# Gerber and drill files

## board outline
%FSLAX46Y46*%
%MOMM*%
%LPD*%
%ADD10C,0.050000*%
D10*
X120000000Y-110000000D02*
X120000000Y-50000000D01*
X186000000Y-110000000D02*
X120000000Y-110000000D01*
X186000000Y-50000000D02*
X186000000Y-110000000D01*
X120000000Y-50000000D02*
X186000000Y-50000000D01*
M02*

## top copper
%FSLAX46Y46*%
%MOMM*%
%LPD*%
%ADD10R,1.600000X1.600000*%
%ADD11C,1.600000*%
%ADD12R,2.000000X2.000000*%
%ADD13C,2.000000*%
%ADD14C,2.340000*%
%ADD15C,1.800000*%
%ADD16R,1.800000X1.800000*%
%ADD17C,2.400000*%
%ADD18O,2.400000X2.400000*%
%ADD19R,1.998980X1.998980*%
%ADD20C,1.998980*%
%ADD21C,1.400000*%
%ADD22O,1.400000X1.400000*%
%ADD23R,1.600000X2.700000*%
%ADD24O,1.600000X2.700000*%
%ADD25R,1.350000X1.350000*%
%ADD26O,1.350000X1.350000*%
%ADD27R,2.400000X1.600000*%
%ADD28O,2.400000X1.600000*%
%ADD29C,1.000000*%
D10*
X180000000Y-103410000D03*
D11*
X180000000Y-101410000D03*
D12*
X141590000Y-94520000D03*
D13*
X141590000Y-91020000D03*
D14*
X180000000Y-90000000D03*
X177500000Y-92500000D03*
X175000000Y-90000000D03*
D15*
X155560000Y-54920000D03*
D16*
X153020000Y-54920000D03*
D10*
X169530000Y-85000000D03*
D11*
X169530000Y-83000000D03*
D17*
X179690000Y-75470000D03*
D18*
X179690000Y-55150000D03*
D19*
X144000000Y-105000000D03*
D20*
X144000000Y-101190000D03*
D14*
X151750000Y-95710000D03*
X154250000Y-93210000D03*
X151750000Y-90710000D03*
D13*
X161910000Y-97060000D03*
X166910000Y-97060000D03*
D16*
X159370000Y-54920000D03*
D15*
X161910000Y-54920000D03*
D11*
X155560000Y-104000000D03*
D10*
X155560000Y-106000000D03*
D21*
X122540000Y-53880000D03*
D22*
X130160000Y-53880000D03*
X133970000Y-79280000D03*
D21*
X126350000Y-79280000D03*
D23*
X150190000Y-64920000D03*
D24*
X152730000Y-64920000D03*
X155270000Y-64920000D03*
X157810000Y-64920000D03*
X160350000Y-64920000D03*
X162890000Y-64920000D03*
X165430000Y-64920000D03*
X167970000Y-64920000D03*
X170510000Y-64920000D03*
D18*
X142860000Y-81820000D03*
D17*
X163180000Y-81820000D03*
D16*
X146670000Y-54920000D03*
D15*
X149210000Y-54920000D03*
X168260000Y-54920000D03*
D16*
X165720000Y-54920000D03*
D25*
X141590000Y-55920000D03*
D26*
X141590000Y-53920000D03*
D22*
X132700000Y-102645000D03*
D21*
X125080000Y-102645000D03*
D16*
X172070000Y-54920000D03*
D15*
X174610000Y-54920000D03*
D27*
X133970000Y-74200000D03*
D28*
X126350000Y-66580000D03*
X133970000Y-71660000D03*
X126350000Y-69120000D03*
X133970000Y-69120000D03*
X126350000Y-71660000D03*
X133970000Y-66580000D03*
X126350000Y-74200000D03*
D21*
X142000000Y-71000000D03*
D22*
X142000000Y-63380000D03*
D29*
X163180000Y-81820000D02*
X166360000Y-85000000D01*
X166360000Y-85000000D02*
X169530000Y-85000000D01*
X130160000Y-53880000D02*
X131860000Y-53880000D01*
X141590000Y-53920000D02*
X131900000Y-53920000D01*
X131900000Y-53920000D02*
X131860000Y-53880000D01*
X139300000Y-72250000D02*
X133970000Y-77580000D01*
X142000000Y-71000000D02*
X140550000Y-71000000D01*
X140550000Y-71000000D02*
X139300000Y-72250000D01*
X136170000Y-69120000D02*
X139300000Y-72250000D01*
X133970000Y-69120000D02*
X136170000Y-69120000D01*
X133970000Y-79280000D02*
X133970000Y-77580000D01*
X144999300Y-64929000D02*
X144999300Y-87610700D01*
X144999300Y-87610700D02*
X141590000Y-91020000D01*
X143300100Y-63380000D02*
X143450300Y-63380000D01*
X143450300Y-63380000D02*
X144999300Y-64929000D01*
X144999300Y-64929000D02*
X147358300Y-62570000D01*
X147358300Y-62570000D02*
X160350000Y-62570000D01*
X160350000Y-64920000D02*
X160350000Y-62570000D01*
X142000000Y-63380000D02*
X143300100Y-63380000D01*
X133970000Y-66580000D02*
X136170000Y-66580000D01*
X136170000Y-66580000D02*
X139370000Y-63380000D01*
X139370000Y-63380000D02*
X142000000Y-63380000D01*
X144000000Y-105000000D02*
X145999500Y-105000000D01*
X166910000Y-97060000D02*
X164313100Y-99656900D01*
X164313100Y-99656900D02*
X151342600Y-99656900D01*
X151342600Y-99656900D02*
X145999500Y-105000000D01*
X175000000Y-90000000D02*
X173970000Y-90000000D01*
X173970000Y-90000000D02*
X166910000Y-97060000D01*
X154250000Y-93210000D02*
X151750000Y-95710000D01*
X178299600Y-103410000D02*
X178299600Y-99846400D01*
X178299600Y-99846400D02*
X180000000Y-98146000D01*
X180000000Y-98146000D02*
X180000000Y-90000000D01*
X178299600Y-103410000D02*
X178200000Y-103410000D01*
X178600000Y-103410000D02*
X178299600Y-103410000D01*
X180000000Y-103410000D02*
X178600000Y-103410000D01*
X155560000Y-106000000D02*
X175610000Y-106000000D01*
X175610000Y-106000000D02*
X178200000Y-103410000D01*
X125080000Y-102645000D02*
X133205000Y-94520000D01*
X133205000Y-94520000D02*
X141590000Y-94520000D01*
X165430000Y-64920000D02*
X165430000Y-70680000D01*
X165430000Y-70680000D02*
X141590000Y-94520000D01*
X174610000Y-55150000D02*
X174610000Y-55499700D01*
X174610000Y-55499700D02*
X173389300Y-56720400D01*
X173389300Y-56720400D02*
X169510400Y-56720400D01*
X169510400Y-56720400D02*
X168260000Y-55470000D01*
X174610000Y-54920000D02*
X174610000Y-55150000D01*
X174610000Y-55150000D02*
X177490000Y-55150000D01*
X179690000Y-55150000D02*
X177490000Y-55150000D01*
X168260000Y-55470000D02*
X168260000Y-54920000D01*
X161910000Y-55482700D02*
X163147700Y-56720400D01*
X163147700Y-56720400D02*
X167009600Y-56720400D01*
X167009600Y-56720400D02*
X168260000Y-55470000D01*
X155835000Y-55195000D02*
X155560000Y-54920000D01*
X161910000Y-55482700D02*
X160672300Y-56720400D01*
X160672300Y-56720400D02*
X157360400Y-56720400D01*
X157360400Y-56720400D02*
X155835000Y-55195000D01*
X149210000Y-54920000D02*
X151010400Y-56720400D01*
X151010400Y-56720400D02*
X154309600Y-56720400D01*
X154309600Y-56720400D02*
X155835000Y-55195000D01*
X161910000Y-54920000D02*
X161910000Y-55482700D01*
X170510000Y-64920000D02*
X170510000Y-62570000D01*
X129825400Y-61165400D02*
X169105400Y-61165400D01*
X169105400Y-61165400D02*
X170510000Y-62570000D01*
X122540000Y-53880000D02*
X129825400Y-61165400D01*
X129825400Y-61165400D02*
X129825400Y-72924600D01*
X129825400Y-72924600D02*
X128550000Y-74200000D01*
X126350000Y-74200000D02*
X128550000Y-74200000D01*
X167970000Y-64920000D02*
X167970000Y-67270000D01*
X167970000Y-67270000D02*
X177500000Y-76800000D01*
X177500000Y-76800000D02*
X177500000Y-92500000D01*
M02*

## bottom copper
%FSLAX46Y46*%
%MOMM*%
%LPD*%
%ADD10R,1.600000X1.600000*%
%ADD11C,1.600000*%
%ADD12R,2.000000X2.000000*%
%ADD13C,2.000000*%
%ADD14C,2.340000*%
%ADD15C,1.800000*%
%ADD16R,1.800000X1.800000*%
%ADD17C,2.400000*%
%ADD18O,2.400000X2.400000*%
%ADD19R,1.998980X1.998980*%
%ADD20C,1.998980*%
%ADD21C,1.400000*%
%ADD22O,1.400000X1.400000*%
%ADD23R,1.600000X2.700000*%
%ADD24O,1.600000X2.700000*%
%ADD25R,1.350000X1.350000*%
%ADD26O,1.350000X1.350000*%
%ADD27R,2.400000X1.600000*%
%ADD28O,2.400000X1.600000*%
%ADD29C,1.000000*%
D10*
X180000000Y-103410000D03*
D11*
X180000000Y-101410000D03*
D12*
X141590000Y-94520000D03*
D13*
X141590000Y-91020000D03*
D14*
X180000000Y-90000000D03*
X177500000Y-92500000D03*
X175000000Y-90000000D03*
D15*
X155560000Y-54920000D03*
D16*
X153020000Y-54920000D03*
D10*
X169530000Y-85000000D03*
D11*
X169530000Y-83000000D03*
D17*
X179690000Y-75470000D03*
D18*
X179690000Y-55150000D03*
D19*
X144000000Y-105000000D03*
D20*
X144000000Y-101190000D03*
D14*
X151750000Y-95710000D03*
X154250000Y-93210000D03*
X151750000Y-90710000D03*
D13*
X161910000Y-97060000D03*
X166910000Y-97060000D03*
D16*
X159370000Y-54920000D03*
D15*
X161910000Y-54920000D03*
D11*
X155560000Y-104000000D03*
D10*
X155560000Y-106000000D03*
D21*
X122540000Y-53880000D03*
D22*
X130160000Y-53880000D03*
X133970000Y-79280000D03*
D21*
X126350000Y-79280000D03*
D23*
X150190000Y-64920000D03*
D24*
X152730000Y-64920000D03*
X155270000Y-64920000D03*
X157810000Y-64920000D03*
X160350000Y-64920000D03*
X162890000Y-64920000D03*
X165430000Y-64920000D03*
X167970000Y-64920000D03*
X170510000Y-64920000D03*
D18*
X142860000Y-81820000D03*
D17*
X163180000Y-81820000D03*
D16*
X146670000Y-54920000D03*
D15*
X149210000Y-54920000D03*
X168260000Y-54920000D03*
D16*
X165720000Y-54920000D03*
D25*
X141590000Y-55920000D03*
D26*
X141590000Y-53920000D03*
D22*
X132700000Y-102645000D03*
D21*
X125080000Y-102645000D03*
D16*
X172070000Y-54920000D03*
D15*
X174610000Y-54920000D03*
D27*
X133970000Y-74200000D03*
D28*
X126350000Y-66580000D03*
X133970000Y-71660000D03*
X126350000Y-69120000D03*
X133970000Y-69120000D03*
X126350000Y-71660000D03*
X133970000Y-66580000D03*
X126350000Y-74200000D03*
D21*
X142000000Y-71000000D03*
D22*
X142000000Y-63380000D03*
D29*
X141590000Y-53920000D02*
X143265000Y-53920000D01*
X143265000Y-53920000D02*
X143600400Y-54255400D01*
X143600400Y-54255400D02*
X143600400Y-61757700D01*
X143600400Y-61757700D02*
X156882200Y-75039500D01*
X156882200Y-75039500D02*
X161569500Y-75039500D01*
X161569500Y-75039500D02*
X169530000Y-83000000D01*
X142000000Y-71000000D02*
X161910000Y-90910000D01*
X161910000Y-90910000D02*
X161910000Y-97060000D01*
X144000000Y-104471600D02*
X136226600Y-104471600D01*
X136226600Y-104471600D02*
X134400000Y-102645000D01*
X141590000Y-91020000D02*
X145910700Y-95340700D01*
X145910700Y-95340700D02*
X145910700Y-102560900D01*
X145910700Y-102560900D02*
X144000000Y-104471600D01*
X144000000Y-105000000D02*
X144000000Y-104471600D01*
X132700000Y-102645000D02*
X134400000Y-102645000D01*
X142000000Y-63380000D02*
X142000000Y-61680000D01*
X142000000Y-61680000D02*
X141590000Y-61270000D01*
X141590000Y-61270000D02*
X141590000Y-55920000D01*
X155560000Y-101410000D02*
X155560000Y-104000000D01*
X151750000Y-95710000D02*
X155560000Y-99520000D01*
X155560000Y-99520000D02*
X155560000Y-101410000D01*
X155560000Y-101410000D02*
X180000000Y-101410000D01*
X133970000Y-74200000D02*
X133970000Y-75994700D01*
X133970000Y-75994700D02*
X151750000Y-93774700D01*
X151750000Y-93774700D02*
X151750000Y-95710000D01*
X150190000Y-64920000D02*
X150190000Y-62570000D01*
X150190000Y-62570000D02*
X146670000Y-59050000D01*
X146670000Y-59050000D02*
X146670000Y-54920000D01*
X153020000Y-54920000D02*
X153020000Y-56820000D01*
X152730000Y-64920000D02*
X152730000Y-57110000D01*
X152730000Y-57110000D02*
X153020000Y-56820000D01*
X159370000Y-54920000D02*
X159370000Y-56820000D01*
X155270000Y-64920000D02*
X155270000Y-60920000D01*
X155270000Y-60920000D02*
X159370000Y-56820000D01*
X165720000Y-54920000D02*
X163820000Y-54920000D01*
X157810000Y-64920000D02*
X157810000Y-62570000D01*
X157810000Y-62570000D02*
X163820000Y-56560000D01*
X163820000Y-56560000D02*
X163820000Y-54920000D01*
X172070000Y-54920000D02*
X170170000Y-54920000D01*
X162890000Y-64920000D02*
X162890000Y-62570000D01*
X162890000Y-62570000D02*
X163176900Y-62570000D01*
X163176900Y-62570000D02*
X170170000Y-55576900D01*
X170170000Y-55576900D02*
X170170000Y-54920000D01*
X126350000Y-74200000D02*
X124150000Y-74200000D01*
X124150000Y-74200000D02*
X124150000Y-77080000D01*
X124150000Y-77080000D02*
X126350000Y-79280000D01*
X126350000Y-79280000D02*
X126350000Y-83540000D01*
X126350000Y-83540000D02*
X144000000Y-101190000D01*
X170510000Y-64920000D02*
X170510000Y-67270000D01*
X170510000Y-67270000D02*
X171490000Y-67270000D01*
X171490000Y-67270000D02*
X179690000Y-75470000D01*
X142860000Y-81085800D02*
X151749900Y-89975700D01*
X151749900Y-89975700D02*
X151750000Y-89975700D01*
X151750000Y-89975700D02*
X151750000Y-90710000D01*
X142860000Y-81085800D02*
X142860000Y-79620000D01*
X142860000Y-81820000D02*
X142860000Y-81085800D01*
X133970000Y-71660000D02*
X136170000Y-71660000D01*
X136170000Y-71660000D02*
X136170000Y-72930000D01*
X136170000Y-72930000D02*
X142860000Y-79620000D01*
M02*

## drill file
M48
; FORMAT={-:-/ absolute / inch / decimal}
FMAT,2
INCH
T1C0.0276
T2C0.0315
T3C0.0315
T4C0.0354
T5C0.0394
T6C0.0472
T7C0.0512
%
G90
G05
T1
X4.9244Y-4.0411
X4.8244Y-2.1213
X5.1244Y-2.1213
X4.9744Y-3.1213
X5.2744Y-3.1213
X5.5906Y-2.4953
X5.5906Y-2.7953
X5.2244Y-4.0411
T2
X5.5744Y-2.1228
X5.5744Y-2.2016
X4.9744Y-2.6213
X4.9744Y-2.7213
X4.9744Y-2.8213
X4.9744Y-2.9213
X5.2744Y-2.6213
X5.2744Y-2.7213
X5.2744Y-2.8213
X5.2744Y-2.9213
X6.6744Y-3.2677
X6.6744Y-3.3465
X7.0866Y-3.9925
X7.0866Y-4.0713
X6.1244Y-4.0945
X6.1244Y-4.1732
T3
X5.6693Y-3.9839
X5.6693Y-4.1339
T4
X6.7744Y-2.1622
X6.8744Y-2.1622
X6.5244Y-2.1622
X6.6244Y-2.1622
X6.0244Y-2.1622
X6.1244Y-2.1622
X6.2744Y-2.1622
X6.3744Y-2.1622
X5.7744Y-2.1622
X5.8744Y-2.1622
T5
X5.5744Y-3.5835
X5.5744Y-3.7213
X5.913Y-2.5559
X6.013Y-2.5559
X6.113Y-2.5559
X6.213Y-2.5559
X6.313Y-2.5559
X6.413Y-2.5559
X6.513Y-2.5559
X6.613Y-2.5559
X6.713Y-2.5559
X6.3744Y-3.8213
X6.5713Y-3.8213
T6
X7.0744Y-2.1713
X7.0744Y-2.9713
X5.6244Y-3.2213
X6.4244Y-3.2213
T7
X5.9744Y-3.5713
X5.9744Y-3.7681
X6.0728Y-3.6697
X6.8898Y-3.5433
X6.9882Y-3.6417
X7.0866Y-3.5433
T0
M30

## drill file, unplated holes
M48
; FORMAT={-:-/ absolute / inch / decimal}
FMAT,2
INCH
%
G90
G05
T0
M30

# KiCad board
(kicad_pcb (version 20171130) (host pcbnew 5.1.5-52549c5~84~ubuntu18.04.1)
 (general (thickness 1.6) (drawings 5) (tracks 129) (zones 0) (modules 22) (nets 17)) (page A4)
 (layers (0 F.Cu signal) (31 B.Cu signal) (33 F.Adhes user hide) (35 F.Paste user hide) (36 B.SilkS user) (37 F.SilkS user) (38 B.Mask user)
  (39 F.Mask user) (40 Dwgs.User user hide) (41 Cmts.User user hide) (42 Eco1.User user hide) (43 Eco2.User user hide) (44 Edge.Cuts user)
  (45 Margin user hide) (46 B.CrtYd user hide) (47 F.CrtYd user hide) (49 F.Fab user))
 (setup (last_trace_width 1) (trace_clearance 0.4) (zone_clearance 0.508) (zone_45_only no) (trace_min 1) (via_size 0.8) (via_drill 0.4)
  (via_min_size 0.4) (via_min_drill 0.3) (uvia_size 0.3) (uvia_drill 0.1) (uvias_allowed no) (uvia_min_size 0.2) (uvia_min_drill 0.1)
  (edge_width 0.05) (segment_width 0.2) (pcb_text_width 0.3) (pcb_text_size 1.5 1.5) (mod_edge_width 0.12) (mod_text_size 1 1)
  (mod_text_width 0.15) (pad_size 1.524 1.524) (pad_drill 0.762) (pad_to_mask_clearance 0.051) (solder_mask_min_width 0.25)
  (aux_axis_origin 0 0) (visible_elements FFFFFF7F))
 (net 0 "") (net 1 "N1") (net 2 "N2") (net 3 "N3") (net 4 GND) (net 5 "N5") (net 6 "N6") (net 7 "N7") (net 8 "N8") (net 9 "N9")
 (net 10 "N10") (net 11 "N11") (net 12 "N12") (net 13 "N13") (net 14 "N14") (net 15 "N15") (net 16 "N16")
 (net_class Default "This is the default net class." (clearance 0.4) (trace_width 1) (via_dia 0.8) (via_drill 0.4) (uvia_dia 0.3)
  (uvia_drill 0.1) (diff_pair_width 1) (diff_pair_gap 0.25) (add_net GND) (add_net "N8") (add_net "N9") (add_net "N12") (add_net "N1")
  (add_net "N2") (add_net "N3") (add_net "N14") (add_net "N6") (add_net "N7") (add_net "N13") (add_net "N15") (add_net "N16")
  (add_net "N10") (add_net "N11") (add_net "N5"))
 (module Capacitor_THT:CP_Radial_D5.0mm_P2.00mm (layer F.Cu) (at 180 103.41 90)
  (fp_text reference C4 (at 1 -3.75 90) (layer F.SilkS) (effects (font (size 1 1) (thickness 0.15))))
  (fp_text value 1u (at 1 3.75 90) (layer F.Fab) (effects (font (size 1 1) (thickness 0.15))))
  (pad 1 thru_hole rect (at 0 0 90) (size 1.6 1.6) (drill 0.8) (layers *.Cu *.Mask) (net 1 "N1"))
  (pad 2 thru_hole circle (at 2 0 90) (size 1.6 1.6) (drill 0.8) (layers *.Cu *.Mask) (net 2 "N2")))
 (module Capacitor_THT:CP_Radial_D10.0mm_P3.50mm (layer F.Cu) (at 141.59 94.52 90)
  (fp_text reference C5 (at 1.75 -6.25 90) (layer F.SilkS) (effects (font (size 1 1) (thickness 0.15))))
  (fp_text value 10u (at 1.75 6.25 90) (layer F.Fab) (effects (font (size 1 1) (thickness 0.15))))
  (pad 1 thru_hole rect (at 0 0 90) (size 2 2) (drill 1) (layers *.Cu *.Mask) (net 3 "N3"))
  (pad 2 thru_hole circle (at 3.5 0 90) (size 2 2) (drill 1) (layers *.Cu *.Mask) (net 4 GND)))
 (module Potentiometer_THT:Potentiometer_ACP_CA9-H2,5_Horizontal (layer F.Cu) (at 180 90 270)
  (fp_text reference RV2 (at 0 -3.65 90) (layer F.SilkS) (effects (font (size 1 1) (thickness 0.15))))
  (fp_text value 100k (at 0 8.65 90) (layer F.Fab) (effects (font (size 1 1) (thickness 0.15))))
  (pad 1 thru_hole circle (at 0 0 270) (size 2.34 2.34) (drill 1.3) (layers *.Cu *.Mask) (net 1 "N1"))
  (pad 2 thru_hole circle (at 2.5 2.5 270) (size 2.34 2.34) (drill 1.3) (layers *.Cu *.Mask) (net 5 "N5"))
  (pad 3 thru_hole circle (at 0 5 270) (size 2.34 2.34) (drill 1.3) (layers *.Cu *.Mask) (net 4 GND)))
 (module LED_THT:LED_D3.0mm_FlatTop (layer F.Cu) (at 153.02 54.92)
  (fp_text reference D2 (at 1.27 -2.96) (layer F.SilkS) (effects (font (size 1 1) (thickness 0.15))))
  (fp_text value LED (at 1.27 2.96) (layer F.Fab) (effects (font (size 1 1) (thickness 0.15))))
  (pad 2 thru_hole circle (at 2.54 0) (size 1.8 1.8) (drill 0.9) (layers *.Cu *.Mask) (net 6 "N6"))
  (pad 1 thru_hole rect (at 0 0) (size 1.8 1.8) (drill 0.9) (layers *.Cu *.Mask) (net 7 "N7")))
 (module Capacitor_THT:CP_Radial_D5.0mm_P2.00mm (layer F.Cu) (at 169.53 85 90)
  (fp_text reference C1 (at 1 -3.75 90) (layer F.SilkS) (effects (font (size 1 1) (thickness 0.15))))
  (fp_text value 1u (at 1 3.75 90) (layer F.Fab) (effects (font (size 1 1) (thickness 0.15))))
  (pad 1 thru_hole rect (at 0 0 90) (size 1.6 1.6) (drill 0.8) (layers *.Cu *.Mask) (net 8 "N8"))
  (pad 2 thru_hole circle (at 2 0 90) (size 1.6 1.6) (drill 0.8) (layers *.Cu *.Mask) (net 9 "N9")))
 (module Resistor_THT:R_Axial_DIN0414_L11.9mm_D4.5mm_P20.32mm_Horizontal (layer F.Cu) (at 179.69 75.47 90)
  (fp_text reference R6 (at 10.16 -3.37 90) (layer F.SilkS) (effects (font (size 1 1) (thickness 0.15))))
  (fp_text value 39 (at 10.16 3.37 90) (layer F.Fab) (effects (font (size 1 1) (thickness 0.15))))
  (pad 1 thru_hole circle (at 0 0 90) (size 2.4 2.4) (drill 1.2) (layers *.Cu *.Mask) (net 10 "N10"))
  (pad 2 thru_hole oval (at 20.32 0 90) (size 2.4 2.4) (drill 1.2) (layers *.Cu *.Mask) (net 6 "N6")))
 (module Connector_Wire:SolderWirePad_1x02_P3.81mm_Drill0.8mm (layer F.Cu) (at 144 105 90)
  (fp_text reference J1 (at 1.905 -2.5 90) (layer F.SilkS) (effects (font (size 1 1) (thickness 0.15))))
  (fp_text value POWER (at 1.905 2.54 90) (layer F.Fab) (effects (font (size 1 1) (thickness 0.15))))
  (pad 1 thru_hole rect (at 0 0 90) (size 1.99898 1.99898) (drill 0.8001) (layers *.Cu *.Mask) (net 4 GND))
  (pad 2 thru_hole circle (at 3.81 0 90) (size 1.99898 1.99898) (drill 0.8001) (layers *.Cu *.Mask) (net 10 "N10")))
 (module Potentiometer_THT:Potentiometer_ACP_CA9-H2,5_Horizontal (layer F.Cu) (at 151.75 90.71)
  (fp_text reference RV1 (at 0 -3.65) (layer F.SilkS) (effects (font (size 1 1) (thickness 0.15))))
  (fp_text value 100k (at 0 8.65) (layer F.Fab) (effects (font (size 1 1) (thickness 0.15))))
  (pad 3 thru_hole circle (at 0 5) (size 2.34 2.34) (drill 1.3) (layers *.Cu *.Mask) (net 2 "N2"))
  (pad 2 thru_hole circle (at 2.5 2.5) (size 2.34 2.34) (drill 1.3) (layers *.Cu *.Mask) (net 2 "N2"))
  (pad 1 thru_hole circle (at 0 0) (size 2.34 2.34) (drill 1.3) (layers *.Cu *.Mask) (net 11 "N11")))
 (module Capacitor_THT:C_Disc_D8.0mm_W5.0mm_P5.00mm (layer F.Cu) (at 161.91 97.06)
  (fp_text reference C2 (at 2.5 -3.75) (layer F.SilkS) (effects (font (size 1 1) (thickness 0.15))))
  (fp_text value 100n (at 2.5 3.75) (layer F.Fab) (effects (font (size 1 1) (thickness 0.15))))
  (pad 1 thru_hole circle (at 0 0) (size 2 2) (drill 1) (layers *.Cu *.Mask) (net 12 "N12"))
  (pad 2 thru_hole circle (at 5 0) (size 2 2) (drill 1) (layers *.Cu *.Mask) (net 4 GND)))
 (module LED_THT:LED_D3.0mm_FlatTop (layer F.Cu) (at 159.37 54.92)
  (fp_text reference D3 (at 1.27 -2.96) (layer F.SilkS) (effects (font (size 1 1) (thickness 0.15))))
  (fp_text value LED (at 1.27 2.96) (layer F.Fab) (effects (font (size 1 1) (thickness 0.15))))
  (pad 1 thru_hole rect (at 0 0) (size 1.8 1.8) (drill 0.9) (layers *.Cu *.Mask) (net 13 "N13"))
  (pad 2 thru_hole circle (at 2.54 0) (size 1.8 1.8) (drill 0.9) (layers *.Cu *.Mask) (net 6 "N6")))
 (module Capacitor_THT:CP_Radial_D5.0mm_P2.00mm (layer F.Cu) (at 155.56 106 90)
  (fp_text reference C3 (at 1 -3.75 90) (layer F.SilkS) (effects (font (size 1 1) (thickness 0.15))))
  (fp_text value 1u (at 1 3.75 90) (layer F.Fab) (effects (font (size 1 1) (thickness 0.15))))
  (pad 2 thru_hole circle (at 2 0 90) (size 1.6 1.6) (drill 0.8) (layers *.Cu *.Mask) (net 2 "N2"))
  (pad 1 thru_hole rect (at 0 0 90) (size 1.6 1.6) (drill 0.8) (layers *.Cu *.Mask) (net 1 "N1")))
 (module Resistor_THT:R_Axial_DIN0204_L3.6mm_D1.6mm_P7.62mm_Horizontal (layer F.Cu) (at 122.54 53.88)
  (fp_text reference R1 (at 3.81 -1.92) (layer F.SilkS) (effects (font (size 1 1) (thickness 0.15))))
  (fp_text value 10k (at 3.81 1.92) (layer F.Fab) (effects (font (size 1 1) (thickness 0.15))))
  (pad 1 thru_hole circle (at 0 0) (size 1.4 1.4) (drill 0.7) (layers *.Cu *.Mask) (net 10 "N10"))
  (pad 2 thru_hole oval (at 7.62 0) (size 1.4 1.4) (drill 0.7) (layers *.Cu *.Mask) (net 9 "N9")))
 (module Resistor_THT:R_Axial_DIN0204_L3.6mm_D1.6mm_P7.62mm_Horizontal (layer F.Cu) (at 126.35 79.28)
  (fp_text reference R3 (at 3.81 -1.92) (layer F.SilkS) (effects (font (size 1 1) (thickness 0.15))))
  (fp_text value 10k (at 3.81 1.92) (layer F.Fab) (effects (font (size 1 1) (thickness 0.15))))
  (pad 2 thru_hole oval (at 7.62 0) (size 1.4 1.4) (drill 0.7) (layers *.Cu *.Mask) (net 12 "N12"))
  (pad 1 thru_hole circle (at 0 0) (size 1.4 1.4) (drill 0.7) (layers *.Cu *.Mask) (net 10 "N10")))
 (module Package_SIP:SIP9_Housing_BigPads (layer F.Cu) (at 150.19 64.92)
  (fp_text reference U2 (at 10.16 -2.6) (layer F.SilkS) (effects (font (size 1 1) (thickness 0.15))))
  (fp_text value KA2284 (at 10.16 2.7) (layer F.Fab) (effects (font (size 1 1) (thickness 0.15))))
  (pad 1 thru_hole rect (at 0 0 90) (size 2.7 1.6) (drill 1) (layers *.Cu *.Mask) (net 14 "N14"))
  (pad 2 thru_hole oval (at 2.54 0 90) (size 2.7 1.6) (drill 1) (layers *.Cu *.Mask) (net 7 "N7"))
  (pad 3 thru_hole oval (at 5.08 0 90) (size 2.7 1.6) (drill 1) (layers *.Cu *.Mask) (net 13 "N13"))
  (pad 4 thru_hole oval (at 7.62 0 90) (size 2.7 1.6) (drill 1) (layers *.Cu *.Mask) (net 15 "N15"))
  (pad 5 thru_hole oval (at 10.16 0 90) (size 2.7 1.6) (drill 1) (layers *.Cu *.Mask) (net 4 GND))
  (pad 6 thru_hole oval (at 12.7 0 90) (size 2.7 1.6) (drill 1) (layers *.Cu *.Mask) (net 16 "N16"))
  (pad 7 thru_hole oval (at 15.24 0 90) (size 2.7 1.6) (drill 1) (layers *.Cu *.Mask) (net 3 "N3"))
  (pad 8 thru_hole oval (at 17.78 0 90) (size 2.7 1.6) (drill 1) (layers *.Cu *.Mask) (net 5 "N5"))
  (pad 9 thru_hole oval (at 20.32 0 90) (size 2.7 1.6) (drill 1) (layers *.Cu *.Mask) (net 10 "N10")))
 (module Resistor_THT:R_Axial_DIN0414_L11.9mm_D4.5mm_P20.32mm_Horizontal (layer F.Cu) (at 163.18 81.82 180)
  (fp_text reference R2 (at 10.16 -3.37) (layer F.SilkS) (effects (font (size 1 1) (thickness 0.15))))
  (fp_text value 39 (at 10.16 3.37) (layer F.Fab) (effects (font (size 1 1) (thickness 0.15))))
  (pad 2 thru_hole oval (at 20.32 0 180) (size 2.4 2.4) (drill 1.2) (layers *.Cu *.Mask) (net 11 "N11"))
  (pad 1 thru_hole circle (at 0 0 180) (size 2.4 2.4) (drill 1.2) (layers *.Cu *.Mask) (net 8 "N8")))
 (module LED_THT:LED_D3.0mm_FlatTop (layer F.Cu) (at 146.67 54.92)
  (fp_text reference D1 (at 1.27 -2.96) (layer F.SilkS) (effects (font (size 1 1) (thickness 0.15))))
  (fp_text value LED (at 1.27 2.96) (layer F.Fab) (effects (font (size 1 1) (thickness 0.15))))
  (pad 1 thru_hole rect (at 0 0) (size 1.8 1.8) (drill 0.9) (layers *.Cu *.Mask) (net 14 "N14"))
  (pad 2 thru_hole circle (at 2.54 0) (size 1.8 1.8) (drill 0.9) (layers *.Cu *.Mask) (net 6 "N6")))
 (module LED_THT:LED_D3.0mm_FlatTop (layer F.Cu) (at 165.72 54.92)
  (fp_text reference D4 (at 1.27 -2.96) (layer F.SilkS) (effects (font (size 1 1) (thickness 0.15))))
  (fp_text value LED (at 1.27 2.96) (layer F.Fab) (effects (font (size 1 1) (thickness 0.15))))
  (pad 2 thru_hole circle (at 2.54 0) (size 1.8 1.8) (drill 0.9) (layers *.Cu *.Mask) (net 6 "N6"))
  (pad 1 thru_hole rect (at 0 0) (size 1.8 1.8) (drill 0.9) (layers *.Cu *.Mask) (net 15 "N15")))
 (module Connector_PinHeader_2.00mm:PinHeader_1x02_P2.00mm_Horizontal (layer F.Cu) (at 141.59 55.92 180)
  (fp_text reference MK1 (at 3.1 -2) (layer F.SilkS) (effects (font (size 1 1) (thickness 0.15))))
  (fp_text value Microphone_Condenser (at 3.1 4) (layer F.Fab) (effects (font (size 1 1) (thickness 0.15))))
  (pad 1 thru_hole rect (at 0 0 180) (size 1.35 1.35) (drill 0.8) (layers *.Cu *.Mask) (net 4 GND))
  (pad 2 thru_hole oval (at 0 2 180) (size 1.35 1.35) (drill 0.8) (layers *.Cu *.Mask) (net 9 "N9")))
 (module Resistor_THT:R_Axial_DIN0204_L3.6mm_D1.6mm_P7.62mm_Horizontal (layer F.Cu) (at 125.08 102.645)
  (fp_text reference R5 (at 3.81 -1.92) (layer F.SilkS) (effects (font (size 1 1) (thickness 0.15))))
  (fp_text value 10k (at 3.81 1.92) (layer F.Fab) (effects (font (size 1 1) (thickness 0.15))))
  (pad 2 thru_hole oval (at 7.62 0) (size 1.4 1.4) (drill 0.7) (layers *.Cu *.Mask) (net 4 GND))
  (pad 1 thru_hole circle (at 0 0) (size 1.4 1.4) (drill 0.7) (layers *.Cu *.Mask) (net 3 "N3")))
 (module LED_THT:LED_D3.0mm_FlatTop (layer F.Cu) (at 172.07 54.92)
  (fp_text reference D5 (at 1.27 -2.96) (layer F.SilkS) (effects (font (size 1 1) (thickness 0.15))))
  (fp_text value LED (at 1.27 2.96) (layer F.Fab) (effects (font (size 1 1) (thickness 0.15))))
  (pad 1 thru_hole rect (at 0 0) (size 1.8 1.8) (drill 0.9) (layers *.Cu *.Mask) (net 16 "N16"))
  (pad 2 thru_hole circle (at 2.54 0) (size 1.8 1.8) (drill 0.9) (layers *.Cu *.Mask) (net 6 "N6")))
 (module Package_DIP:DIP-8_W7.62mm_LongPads (layer F.Cu) (at 133.97 74.2 180)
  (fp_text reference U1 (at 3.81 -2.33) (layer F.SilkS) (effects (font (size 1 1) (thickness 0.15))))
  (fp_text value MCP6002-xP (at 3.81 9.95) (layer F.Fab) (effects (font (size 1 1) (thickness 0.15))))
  (pad 1 thru_hole rect (at 0 0 180) (size 2.4 1.6) (drill 0.8) (layers *.Cu *.Mask) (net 2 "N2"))
  (pad 5 thru_hole oval (at 7.62 7.62 180) (size 2.4 1.6) (drill 0.8) (layers *.Cu *.Mask))
  (pad 2 thru_hole oval (at 0 2.54 180) (size 2.4 1.6) (drill 0.8) (layers *.Cu *.Mask) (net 11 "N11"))
  (pad 6 thru_hole oval (at 7.62 5.08 180) (size 2.4 1.6) (drill 0.8) (layers *.Cu *.Mask))
  (pad 3 thru_hole oval (at 0 5.08 180) (size 2.4 1.6) (drill 0.8) (layers *.Cu *.Mask) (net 12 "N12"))
  (pad 7 thru_hole oval (at 7.62 2.54 180) (size 2.4 1.6) (drill 0.8) (layers *.Cu *.Mask))
  (pad 4 thru_hole oval (at 0 7.62 180) (size 2.4 1.6) (drill 0.8) (layers *.Cu *.Mask) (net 4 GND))
  (pad 8 thru_hole oval (at 7.62 0 180) (size 2.4 1.6) (drill 0.8) (layers *.Cu *.Mask) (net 10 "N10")))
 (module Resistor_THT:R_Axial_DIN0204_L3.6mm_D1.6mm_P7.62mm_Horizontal (layer F.Cu) (at 142 71 90)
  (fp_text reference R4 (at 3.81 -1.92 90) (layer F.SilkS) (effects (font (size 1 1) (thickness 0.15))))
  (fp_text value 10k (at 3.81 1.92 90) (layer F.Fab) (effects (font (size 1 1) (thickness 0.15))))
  (pad 1 thru_hole circle (at 0 0 90) (size 1.4 1.4) (drill 0.7) (layers *.Cu *.Mask) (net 12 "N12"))
  (pad 2 thru_hole oval (at 7.62 0 90) (size 1.4 1.4) (drill 0.7) (layers *.Cu *.Mask) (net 4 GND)))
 (gr_line (start 120 110) (end 120 50) (layer Edge.Cuts) (width 0.05))
 (gr_line (start 186 110) (end 120 110) (layer Edge.Cuts) (width 0.05))
 (gr_line (start 186 50) (end 186 110) (layer Edge.Cuts) (width 0.05))
 (gr_line (start 120 50) (end 186 50) (layer Edge.Cuts) (width 0.05))
 (segment (start 163.18 81.82) (end 166.36 85) (width 1) (layer F.Cu) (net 8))
 (segment (start 166.36 85) (end 169.53 85) (width 1) (layer F.Cu) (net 8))
 (segment (start 141.59 53.92) (end 143.265 53.92) (width 1) (layer B.Cu) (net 9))
 (segment (start 143.265 53.92) (end 143.6004 54.2554) (width 1) (layer B.Cu) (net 9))
 (segment (start 143.6004 54.2554) (end 143.6004 61.7577) (width 1) (layer B.Cu) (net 9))
 (segment (start 143.6004 61.7577) (end 156.8822 75.0395) (width 1) (layer B.Cu) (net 9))
 (segment (start 156.8822 75.0395) (end 161.5695 75.0395) (width 1) (layer B.Cu) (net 9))
 (segment (start 161.5695 75.0395) (end 169.53 83) (width 1) (layer B.Cu) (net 9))
 (segment (start 130.16 53.88) (end 131.86 53.88) (width 1) (layer F.Cu) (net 9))
 (segment (start 141.59 53.92) (end 131.9 53.92) (width 1) (layer F.Cu) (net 9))
 (segment (start 131.9 53.92) (end 131.86 53.88) (width 1) (layer F.Cu) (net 9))
 (segment (start 142 71) (end 161.91 90.91) (width 1) (layer B.Cu) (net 12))
 (segment (start 161.91 90.91) (end 161.91 97.06) (width 1) (layer B.Cu) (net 12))
 (segment (start 139.3 72.25) (end 133.97 77.58) (width 1) (layer F.Cu) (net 12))
 (segment (start 142 71) (end 140.55 71) (width 1) (layer F.Cu) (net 12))
 (segment (start 140.55 71) (end 139.3 72.25) (width 1) (layer F.Cu) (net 12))
 (segment (start 136.17 69.12) (end 139.3 72.25) (width 1) (layer F.Cu) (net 12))
 (segment (start 133.97 69.12) (end 136.17 69.12) (width 1) (layer F.Cu) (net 12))
 (segment (start 133.97 79.28) (end 133.97 77.58) (width 1) (layer F.Cu) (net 12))
 (segment (start 144.9993 64.929) (end 144.9993 87.6107) (width 1) (layer F.Cu) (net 4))
 (segment (start 144.9993 87.6107) (end 141.59 91.02) (width 1) (layer F.Cu) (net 4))
 (segment (start 143.3001 63.38) (end 143.4503 63.38) (width 1) (layer F.Cu) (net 4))
 (segment (start 143.4503 63.38) (end 144.9993 64.929) (width 1) (layer F.Cu) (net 4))
 (segment (start 144.9993 64.929) (end 147.3583 62.57) (width 1) (layer F.Cu) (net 4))
 (segment (start 147.3583 62.57) (end 160.35 62.57) (width 1) (layer F.Cu) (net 4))
 (segment (start 160.35 64.92) (end 160.35 62.57) (width 1) (layer F.Cu) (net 4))
 (segment (start 142 63.38) (end 143.3001 63.38) (width 1) (layer F.Cu) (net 4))
 (segment (start 144 104.4716) (end 136.2266 104.4716) (width 1) (layer B.Cu) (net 4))
 (segment (start 136.2266 104.4716) (end 134.4 102.645) (width 1) (layer B.Cu) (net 4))
 (segment (start 141.59 91.02) (end 145.9107 95.3407) (width 1) (layer B.Cu) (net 4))
 (segment (start 145.9107 95.3407) (end 145.9107 102.5609) (width 1) (layer B.Cu) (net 4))
 (segment (start 145.9107 102.5609) (end 144 104.4716) (width 1) (layer B.Cu) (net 4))
 (segment (start 144 105) (end 144 104.4716) (width 1) (layer B.Cu) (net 4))
 (segment (start 132.7 102.645) (end 134.4 102.645) (width 1) (layer B.Cu) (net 4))
 (segment (start 142 63.38) (end 142 61.68) (width 1) (layer B.Cu) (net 4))
 (segment (start 142 61.68) (end 141.59 61.27) (width 1) (layer B.Cu) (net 4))
 (segment (start 141.59 61.27) (end 141.59 55.92) (width 1) (layer B.Cu) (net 4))
 (segment (start 133.97 66.58) (end 136.17 66.58) (width 1) (layer F.Cu) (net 4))
 (segment (start 136.17 66.58) (end 139.37 63.38) (width 1) (layer F.Cu) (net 4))
 (segment (start 139.37 63.38) (end 142 63.38) (width 1) (layer F.Cu) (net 4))
 (segment (start 144 105) (end 145.9995 105) (width 1) (layer F.Cu) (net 4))
 (segment (start 166.91 97.06) (end 164.3131 99.6569) (width 1) (layer F.Cu) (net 4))
 (segment (start 164.3131 99.6569) (end 151.3426 99.6569) (width 1) (layer F.Cu) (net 4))
 (segment (start 151.3426 99.6569) (end 145.9995 105) (width 1) (layer F.Cu) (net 4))
 (segment (start 175 90) (end 173.97 90) (width 1) (layer F.Cu) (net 4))
 (segment (start 173.97 90) (end 166.91 97.06) (width 1) (layer F.Cu) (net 4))
 (segment (start 155.56 101.41) (end 155.56 104) (width 1) (layer B.Cu) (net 2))
 (segment (start 151.75 95.71) (end 155.56 99.52) (width 1) (layer B.Cu) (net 2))
 (segment (start 155.56 99.52) (end 155.56 101.41) (width 1) (layer B.Cu) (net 2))
 (segment (start 155.56 101.41) (end 180 101.41) (width 1) (layer B.Cu) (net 2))
 (segment (start 133.97 74.2) (end 133.97 75.9947) (width 1) (layer B.Cu) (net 2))
 (segment (start 133.97 75.9947) (end 151.75 93.7747) (width 1) (layer B.Cu) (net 2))
 (segment (start 151.75 93.7747) (end 151.75 95.71) (width 1) (layer B.Cu) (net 2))
 (segment (start 154.25 93.21) (end 151.75 95.71) (width 1) (layer F.Cu) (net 2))
 (segment (start 178.2996 103.41) (end 178.2996 99.8464) (width 1) (layer F.Cu) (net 1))
 (segment (start 178.2996 99.8464) (end 180 98.146) (width 1) (layer F.Cu) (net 1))
 (segment (start 180 98.146) (end 180 90) (width 1) (layer F.Cu) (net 1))
 (segment (start 178.2996 103.41) (end 178.2 103.41) (width 1) (layer F.Cu) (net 1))
 (segment (start 178.6 103.41) (end 178.2996 103.41) (width 1) (layer F.Cu) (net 1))
 (segment (start 180 103.41) (end 178.6 103.41) (width 1) (layer F.Cu) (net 1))
 (segment (start 155.56 106) (end 175.61 106) (width 1) (layer F.Cu) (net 1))
 (segment (start 175.61 106) (end 178.2 103.41) (width 1) (layer F.Cu) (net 1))
 (segment (start 125.08 102.645) (end 133.205 94.52) (width 1) (layer F.Cu) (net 3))
 (segment (start 133.205 94.52) (end 141.59 94.52) (width 1) (layer F.Cu) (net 3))
 (segment (start 165.43 64.92) (end 165.43 70.68) (width 1) (layer F.Cu) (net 3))
 (segment (start 165.43 70.68) (end 141.59 94.52) (width 1) (layer F.Cu) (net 3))
 (segment (start 150.19 64.92) (end 150.19 62.57) (width 1) (layer B.Cu) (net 14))
 (segment (start 150.19 62.57) (end 146.67 59.05) (width 1) (layer B.Cu) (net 14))
 (segment (start 146.67 59.05) (end 146.67 54.92) (width 1) (layer B.Cu) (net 14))
 (segment (start 174.61 55.15) (end 174.61 55.4997) (width 1) (layer F.Cu) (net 6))
 (segment (start 174.61 55.4997) (end 173.3893 56.7204) (width 1) (layer F.Cu) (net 6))
 (segment (start 173.3893 56.7204) (end 169.5104 56.7204) (width 1) (layer F.Cu) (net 6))
 (segment (start 169.5104 56.7204) (end 168.26 55.47) (width 1) (layer F.Cu) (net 6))
 (segment (start 174.61 54.92) (end 174.61 55.15) (width 1) (layer F.Cu) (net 6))
 (segment (start 174.61 55.15) (end 177.49 55.15) (width 1) (layer F.Cu) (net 6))
 (segment (start 179.69 55.15) (end 177.49 55.15) (width 1) (layer F.Cu) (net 6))
 (segment (start 168.26 55.47) (end 168.26 54.92) (width 1) (layer F.Cu) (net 6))
 (segment (start 161.91 55.4827) (end 163.1477 56.7204) (width 1) (layer F.Cu) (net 6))
 (segment (start 163.1477 56.7204) (end 167.0096 56.7204) (width 1) (layer F.Cu) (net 6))
 (segment (start 167.0096 56.7204) (end 168.26 55.47) (width 1) (layer F.Cu) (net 6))
 (segment (start 155.835 55.195) (end 155.56 54.92) (width 1) (layer F.Cu) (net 6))
 (segment (start 161.91 55.4827) (end 160.6723 56.7204) (width 1) (layer F.Cu) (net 6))
 (segment (start 160.6723 56.7204) (end 157.3604 56.7204) (width 1) (layer F.Cu) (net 6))
 (segment (start 157.3604 56.7204) (end 155.835 55.195) (width 1) (layer F.Cu) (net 6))
 (segment (start 149.21 54.92) (end 151.0104 56.7204) (width 1) (layer F.Cu) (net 6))
 (segment (start 151.0104 56.7204) (end 154.3096 56.7204) (width 1) (layer F.Cu) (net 6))
 (segment (start 154.3096 56.7204) (end 155.835 55.195) (width 1) (layer F.Cu) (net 6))
 (segment (start 161.91 54.92) (end 161.91 55.4827) (width 1) (layer F.Cu) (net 6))
 (segment (start 153.02 54.92) (end 153.02 56.82) (width 1) (layer B.Cu) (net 7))
 (segment (start 152.73 64.92) (end 152.73 57.11) (width 1) (layer B.Cu) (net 7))
 (segment (start 152.73 57.11) (end 153.02 56.82) (width 1) (layer B.Cu) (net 7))
 (segment (start 159.37 54.92) (end 159.37 56.82) (width 1) (layer B.Cu) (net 13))
 (segment (start 155.27 64.92) (end 155.27 60.92) (width 1) (layer B.Cu) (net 13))
 (segment (start 155.27 60.92) (end 159.37 56.82) (width 1) (layer B.Cu) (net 13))
 (segment (start 165.72 54.92) (end 163.82 54.92) (width 1) (layer B.Cu) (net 15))
 (segment (start 157.81 64.92) (end 157.81 62.57) (width 1) (layer B.Cu) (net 15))
 (segment (start 157.81 62.57) (end 163.82 56.56) (width 1) (layer B.Cu) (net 15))
 (segment (start 163.82 56.56) (end 163.82 54.92) (width 1) (layer B.Cu) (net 15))
 (segment (start 172.07 54.92) (end 170.17 54.92) (width 1) (layer B.Cu) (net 16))
 (segment (start 162.89 64.92) (end 162.89 62.57) (width 1) (layer B.Cu) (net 16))
 (segment (start 162.89 62.57) (end 163.1769 62.57) (width 1) (layer B.Cu) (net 16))
 (segment (start 163.1769 62.57) (end 170.17 55.5769) (width 1) (layer B.Cu) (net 16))
 (segment (start 170.17 55.5769) (end 170.17 54.92) (width 1) (layer B.Cu) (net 16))
 (segment (start 170.51 64.92) (end 170.51 62.57) (width 1) (layer F.Cu) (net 10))
 (segment (start 129.8254 61.1654) (end 169.1054 61.1654) (width 1) (layer F.Cu) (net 10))
 (segment (start 169.1054 61.1654) (end 170.51 62.57) (width 1) (layer F.Cu) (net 10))
 (segment (start 122.54 53.88) (end 129.8254 61.1654) (width 1) (layer F.Cu) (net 10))
 (segment (start 129.8254 61.1654) (end 129.8254 72.9246) (width 1) (layer F.Cu) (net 10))
 (segment (start 129.8254 72.9246) (end 128.55 74.2) (width 1) (layer F.Cu) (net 10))
 (segment (start 126.35 74.2) (end 128.55 74.2) (width 1) (layer F.Cu) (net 10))
 (segment (start 126.35 74.2) (end 124.15 74.2) (width 1) (layer B.Cu) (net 10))
 (segment (start 124.15 74.2) (end 124.15 77.08) (width 1) (layer B.Cu) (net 10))
 (segment (start 124.15 77.08) (end 126.35 79.28) (width 1) (layer B.Cu) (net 10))
 (segment (start 126.35 79.28) (end 126.35 83.54) (width 1) (layer B.Cu) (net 10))
 (segment (start 126.35 83.54) (end 144 101.19) (width 1) (layer B.Cu) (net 10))
 (segment (start 170.51 64.92) (end 170.51 67.27) (width 1) (layer B.Cu) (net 10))
 (segment (start 170.51 67.27) (end 171.49 67.27) (width 1) (layer B.Cu) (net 10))
 (segment (start 171.49 67.27) (end 179.69 75.47) (width 1) (layer B.Cu) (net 10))
 (segment (start 142.86 81.0858) (end 151.7499 89.9757) (width 1) (layer B.Cu) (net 11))
 (segment (start 151.7499 89.9757) (end 151.75 89.9757) (width 1) (layer B.Cu) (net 11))
 (segment (start 151.75 89.9757) (end 151.75 90.71) (width 1) (layer B.Cu) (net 11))
 (segment (start 142.86 81.0858) (end 142.86 79.62) (width 1) (layer B.Cu) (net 11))
 (segment (start 142.86 81.82) (end 142.86 81.0858) (width 1) (layer B.Cu) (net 11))
 (segment (start 133.97 71.66) (end 136.17 71.66) (width 1) (layer B.Cu) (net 11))
 (segment (start 136.17 71.66) (end 136.17 72.93) (width 1) (layer B.Cu) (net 11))
 (segment (start 136.17 72.93) (end 142.86 79.62) (width 1) (layer B.Cu) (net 11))
 (segment (start 167.97 64.92) (end 167.97 67.27) (width 1) (layer F.Cu) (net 5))
 (segment (start 167.97 67.27) (end 177.5 76.8) (width 1) (layer F.Cu) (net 5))
 (segment (start 177.5 76.8) (end 177.5 92.5) (width 1) (layer F.Cu) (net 5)))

